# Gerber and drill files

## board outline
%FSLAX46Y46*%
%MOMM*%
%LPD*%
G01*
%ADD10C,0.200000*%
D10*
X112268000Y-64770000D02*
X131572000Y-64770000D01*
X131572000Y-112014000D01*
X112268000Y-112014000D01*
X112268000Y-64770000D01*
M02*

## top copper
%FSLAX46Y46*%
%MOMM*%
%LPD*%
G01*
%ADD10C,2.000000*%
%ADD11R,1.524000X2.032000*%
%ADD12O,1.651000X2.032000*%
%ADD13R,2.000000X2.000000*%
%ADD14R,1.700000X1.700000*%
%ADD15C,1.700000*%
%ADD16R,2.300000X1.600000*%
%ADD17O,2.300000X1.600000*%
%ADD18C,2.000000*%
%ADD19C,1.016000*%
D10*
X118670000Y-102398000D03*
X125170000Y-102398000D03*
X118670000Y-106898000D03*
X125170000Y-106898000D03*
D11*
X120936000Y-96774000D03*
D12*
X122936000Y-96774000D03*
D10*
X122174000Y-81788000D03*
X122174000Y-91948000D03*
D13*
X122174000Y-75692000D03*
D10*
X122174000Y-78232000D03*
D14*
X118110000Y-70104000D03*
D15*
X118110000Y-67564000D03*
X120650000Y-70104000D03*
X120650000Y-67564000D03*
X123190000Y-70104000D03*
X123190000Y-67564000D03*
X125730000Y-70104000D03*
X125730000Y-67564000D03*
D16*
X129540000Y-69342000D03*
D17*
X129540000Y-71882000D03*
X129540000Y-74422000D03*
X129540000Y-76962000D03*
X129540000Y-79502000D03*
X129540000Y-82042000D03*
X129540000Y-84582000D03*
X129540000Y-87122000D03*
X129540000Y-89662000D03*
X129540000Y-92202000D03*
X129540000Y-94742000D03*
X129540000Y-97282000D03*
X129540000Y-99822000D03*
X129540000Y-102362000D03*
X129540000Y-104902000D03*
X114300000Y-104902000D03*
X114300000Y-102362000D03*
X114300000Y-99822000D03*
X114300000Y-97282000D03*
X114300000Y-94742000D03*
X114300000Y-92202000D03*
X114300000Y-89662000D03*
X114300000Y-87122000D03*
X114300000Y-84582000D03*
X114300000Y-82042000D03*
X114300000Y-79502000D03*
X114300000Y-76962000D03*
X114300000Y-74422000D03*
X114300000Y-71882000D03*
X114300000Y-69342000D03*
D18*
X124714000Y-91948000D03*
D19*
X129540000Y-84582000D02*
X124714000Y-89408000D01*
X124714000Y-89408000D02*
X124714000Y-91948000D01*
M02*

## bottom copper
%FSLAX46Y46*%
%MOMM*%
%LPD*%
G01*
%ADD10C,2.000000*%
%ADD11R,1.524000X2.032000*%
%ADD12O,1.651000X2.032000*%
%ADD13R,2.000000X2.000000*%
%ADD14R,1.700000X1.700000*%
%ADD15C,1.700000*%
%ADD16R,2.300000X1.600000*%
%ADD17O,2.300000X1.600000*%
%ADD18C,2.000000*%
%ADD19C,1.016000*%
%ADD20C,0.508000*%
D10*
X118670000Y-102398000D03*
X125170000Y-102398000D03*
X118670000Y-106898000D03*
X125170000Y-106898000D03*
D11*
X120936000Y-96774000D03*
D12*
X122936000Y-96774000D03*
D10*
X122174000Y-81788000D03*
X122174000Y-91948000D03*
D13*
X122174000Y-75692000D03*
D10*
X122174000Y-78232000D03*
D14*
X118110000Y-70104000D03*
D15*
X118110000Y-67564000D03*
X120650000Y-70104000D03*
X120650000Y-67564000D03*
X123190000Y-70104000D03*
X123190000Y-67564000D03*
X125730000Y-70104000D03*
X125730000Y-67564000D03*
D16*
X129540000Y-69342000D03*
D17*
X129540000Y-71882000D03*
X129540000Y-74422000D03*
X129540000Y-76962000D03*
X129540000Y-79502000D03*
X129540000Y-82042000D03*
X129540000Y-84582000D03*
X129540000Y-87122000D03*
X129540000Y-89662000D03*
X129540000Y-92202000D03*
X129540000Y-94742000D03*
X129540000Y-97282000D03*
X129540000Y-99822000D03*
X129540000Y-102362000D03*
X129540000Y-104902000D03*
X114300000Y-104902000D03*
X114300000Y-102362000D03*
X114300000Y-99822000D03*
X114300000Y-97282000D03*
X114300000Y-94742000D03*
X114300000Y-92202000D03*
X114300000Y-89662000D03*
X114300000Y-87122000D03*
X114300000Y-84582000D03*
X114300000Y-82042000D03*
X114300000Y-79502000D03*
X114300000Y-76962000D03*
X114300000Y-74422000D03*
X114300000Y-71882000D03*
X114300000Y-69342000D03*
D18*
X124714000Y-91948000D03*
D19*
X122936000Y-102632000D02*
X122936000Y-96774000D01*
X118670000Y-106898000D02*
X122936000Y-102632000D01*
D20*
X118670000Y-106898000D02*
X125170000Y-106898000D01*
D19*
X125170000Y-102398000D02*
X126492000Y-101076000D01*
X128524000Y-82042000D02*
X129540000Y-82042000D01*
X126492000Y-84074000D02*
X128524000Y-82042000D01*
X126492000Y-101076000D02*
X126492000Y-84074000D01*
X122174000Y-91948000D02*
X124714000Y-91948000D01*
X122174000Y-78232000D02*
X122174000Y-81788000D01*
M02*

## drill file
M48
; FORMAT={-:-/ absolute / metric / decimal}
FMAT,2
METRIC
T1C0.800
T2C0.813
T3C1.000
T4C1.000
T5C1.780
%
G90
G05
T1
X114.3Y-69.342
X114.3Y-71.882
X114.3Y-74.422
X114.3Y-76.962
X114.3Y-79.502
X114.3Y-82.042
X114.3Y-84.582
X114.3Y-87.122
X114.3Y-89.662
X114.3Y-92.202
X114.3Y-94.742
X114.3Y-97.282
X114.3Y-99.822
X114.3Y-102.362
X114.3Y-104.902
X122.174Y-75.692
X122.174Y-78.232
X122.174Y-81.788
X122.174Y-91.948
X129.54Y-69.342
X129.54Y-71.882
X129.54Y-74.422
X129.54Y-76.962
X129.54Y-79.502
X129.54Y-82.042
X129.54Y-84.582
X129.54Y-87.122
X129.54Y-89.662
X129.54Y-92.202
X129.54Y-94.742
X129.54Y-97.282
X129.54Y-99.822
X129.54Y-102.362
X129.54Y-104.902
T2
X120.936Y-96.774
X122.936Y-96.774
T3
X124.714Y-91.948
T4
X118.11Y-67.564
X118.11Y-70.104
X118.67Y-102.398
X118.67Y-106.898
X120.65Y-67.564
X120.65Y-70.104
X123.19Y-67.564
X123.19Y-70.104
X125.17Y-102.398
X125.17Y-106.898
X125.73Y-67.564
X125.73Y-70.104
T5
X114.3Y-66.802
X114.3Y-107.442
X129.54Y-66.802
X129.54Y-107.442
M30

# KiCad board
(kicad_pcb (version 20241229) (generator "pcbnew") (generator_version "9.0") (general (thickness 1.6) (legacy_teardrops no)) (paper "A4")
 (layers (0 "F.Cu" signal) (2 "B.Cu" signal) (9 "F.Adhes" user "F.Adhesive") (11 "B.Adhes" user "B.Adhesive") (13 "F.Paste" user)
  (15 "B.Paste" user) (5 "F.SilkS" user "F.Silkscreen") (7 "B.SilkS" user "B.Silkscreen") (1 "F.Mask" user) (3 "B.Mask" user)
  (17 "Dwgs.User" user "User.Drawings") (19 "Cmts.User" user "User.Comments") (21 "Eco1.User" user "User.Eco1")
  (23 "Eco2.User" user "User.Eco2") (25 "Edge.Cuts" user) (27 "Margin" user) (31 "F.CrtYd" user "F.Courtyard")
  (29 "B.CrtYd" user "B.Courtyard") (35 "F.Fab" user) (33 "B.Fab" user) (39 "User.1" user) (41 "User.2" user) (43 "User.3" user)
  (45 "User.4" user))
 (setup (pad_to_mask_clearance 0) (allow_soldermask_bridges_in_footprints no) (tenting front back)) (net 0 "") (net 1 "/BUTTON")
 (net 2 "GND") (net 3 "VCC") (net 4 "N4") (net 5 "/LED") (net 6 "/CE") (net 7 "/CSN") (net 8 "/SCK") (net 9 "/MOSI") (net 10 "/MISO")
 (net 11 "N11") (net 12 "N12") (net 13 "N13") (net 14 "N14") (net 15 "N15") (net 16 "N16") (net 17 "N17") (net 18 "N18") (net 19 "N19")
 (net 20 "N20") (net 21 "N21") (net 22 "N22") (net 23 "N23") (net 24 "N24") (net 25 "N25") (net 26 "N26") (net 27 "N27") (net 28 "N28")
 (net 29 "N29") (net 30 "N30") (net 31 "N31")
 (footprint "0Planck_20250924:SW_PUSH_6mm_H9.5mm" (layer "F.Cu") (at 118.67 102.398)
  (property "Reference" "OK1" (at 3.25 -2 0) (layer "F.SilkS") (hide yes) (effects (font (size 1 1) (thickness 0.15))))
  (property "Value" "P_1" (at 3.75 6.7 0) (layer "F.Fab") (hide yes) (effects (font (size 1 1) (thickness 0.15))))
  (pad "1" thru_hole circle (at 0 0) (size 2 2) (drill 1) (layers "*.Cu" "*.Mask") (remove_unused_layers no) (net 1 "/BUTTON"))
  (pad "1" thru_hole circle (at 6.5 0) (size 2 2) (drill 1) (layers "*.Cu" "*.Mask") (remove_unused_layers no) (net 1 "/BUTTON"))
  (pad "2" thru_hole circle (at 0 4.5) (size 2 2) (drill 1) (layers "*.Cu" "*.Mask") (remove_unused_layers no) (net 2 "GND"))
  (pad "2" thru_hole circle (at 6.5 4.5) (size 2 2) (drill 1) (layers "*.Cu" "*.Mask") (remove_unused_layers no) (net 2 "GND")))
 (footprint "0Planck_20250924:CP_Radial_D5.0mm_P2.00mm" (layer "F.Cu") (at 120.936 96.774)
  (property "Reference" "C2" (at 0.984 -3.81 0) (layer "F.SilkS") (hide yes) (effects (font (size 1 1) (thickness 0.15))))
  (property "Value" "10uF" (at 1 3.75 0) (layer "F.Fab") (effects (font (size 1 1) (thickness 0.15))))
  (pad "1" thru_hole rect (at 0 0) (size 1.524 2.032) (drill 0.8128) (layers "*.Cu" "*.Mask") (remove_unused_layers no) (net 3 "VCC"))
  (pad "2" thru_hole oval (at 2 0) (size 1.651 2.032) (drill 0.8128) (layers "*.Cu" "*.Mask") (remove_unused_layers no) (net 2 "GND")))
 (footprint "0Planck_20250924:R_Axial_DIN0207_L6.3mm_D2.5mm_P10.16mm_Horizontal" (layer "F.Cu") (at 122.174 81.788 -90)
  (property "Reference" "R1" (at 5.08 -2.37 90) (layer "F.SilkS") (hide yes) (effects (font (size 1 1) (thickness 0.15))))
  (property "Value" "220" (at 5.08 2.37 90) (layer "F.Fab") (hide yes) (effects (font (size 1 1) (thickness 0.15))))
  (pad "1" thru_hole circle (at 0 0 270) (size 2 2) (drill 0.8) (layers "*.Cu" "*.Mask") (remove_unused_layers no) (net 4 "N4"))
  (pad "2" thru_hole circle (at 10.16 0 270) (size 2 2) (drill 0.8) (layers "*.Cu" "*.Mask") (remove_unused_layers no) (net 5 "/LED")))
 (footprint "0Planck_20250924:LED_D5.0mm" (layer "F.Cu") (at 122.174 75.692 -90)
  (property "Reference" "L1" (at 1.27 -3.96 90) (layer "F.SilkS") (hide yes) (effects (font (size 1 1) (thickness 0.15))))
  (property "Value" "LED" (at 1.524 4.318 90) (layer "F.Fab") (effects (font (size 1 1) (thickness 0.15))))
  (pad "1" thru_hole rect (at 0 0 270) (size 2 2) (drill 0.8) (layers "*.Cu" "*.Mask") (remove_unused_layers no) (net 2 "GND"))
  (pad "2" thru_hole circle (at 2.54 0 270) (size 2 2) (drill 0.8) (layers "*.Cu" "*.Mask") (remove_unused_layers no) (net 4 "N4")))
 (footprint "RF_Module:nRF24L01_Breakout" (layer "F.Cu") (at 118.11 70.104 90)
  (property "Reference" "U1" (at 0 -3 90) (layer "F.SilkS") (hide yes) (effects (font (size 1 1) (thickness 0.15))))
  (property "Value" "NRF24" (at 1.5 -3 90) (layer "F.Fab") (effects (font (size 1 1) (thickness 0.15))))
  (pad "1" thru_hole rect (at 0 0 90) (size 1.7 1.7) (drill 1) (layers "*.Cu" "*.Mask") (remove_unused_layers no) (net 2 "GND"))
  (pad "2" thru_hole circle (at 2.54 0 90) (size 1.7 1.7) (drill 1) (layers "*.Cu" "*.Mask") (remove_unused_layers no) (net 3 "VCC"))
  (pad "3" thru_hole circle (at 0 2.54 90) (size 1.7 1.7) (drill 1) (layers "*.Cu" "*.Mask") (remove_unused_layers no) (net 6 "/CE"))
  (pad "4" thru_hole circle (at 2.54 2.54 90) (size 1.7 1.7) (drill 1) (layers "*.Cu" "*.Mask") (remove_unused_layers no) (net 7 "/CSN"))
  (pad "5" thru_hole circle (at 0 5.08 90) (size 1.7 1.7) (drill 1) (layers "*.Cu" "*.Mask") (remove_unused_layers no) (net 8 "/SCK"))
  (pad "6" thru_hole circle (at 2.54 5.08 90) (size 1.7 1.7) (drill 1) (layers "*.Cu" "*.Mask") (remove_unused_layers no) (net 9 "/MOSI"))
  (pad "7" thru_hole circle (at 0 7.62 90) (size 1.7 1.7) (drill 1) (layers "*.Cu" "*.Mask") (remove_unused_layers no) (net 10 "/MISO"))
  (pad "8" thru_hole circle (at 2.54 7.62 90) (size 1.7 1.7) (drill 1) (layers "*.Cu" "*.Mask") (remove_unused_layers no) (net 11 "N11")))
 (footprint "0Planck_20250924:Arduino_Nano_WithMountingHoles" (layer "B.Cu") (at 129.54 69.342 180)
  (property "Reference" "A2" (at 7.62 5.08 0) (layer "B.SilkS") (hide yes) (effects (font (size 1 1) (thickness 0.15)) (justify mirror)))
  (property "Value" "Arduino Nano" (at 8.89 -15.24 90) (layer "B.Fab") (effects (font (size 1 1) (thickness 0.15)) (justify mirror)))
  (pad "" np_thru_hole circle (at 0 -38.1 180) (size 1.78 1.78) (drill 1.78) (layers "*.Cu" "*.Mask"))
  (pad "" np_thru_hole circle (at 0 2.54 180) (size 1.78 1.78) (drill 1.78) (layers "*.Cu" "*.Mask"))
  (pad "" np_thru_hole circle (at 15.24 -38.1 180) (size 1.78 1.78) (drill 1.78) (layers "*.Cu" "*.Mask"))
  (pad "" np_thru_hole circle (at 15.24 2.54 180) (size 1.78 1.78) (drill 1.78) (layers "*.Cu" "*.Mask"))
  (pad "1" thru_hole rect (at 0 0 180) (size 2.3 1.6) (drill 0.8) (layers "*.Cu" "*.Mask") (remove_unused_layers no) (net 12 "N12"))
  (pad "2" thru_hole oval (at 0 -2.54 180) (size 2.3 1.6) (drill 0.8) (layers "*.Cu" "*.Mask") (remove_unused_layers no) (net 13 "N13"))
  (pad "3" thru_hole oval (at 0 -5.08 180) (size 2.3 1.6) (drill 0.8) (layers "*.Cu" "*.Mask") (remove_unused_layers no) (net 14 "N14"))
  (pad "4" thru_hole oval (at 0 -7.62 180) (size 2.3 1.6) (drill 0.8) (layers "*.Cu" "*.Mask") (remove_unused_layers no) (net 2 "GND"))
  (pad "5" thru_hole oval (at 0 -10.16 180) (size 2.3 1.6) (drill 0.8) (layers "*.Cu" "*.Mask") (remove_unused_layers no) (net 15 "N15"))
  (pad "6" thru_hole oval (at 0 -12.7 180) (size 2.3 1.6) (drill 0.8) (layers "*.Cu" "*.Mask") (remove_unused_layers no) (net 1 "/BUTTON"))
  (pad "7" thru_hole oval (at 0 -15.24 180) (size 2.3 1.6) (drill 0.8) (layers "*.Cu" "*.Mask") (remove_unused_layers no) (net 5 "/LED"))
  (pad "8" thru_hole oval (at 0 -17.78 180) (size 2.3 1.6) (drill 0.8) (layers "*.Cu" "*.Mask") (remove_unused_layers no) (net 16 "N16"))
  (pad "9" thru_hole oval (at 0 -20.32 180) (size 2.3 1.6) (drill 0.8) (layers "*.Cu" "*.Mask") (remove_unused_layers no) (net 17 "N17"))
  (pad "10" thru_hole oval (at 0 -22.86 180) (size 2.3 1.6) (drill 0.8) (layers "*.Cu" "*.Mask") (remove_unused_layers no) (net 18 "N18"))
  (pad "11" thru_hole oval (at 0 -25.4 180) (size 2.3 1.6) (drill 0.8) (layers "*.Cu" "*.Mask") (remove_unused_layers no) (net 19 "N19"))
  (pad "12" thru_hole oval (at 0 -27.94 180) (size 2.3 1.6) (drill 0.8) (layers "*.Cu" "*.Mask") (remove_unused_layers no) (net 6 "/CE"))
  (pad "13" thru_hole oval (at 0 -30.48 180) (size 2.3 1.6) (drill 0.8) (layers "*.Cu" "*.Mask") (remove_unused_layers no) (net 7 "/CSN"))
  (pad "14" thru_hole oval (at 0 -33.02 180) (size 2.3 1.6) (drill 0.8) (layers "*.Cu" "*.Mask") (remove_unused_layers no) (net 9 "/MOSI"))
  (pad "15" thru_hole oval (at 0 -35.56 180) (size 2.3 1.6) (drill 0.8) (layers "*.Cu" "*.Mask") (remove_unused_layers no) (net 10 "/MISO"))
  (pad "16" thru_hole oval (at 15.24 -35.56 180) (size 2.3 1.6) (drill 0.8) (layers "*.Cu" "*.Mask") (remove_unused_layers no)
   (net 8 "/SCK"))
  (pad "17" thru_hole oval (at 15.24 -33.02 180) (size 2.3 1.6) (drill 0.8) (layers "*.Cu" "*.Mask") (remove_unused_layers no) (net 3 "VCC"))
  (pad "18" thru_hole oval (at 15.24 -30.48 180) (size 2.3 1.6) (drill 0.8) (layers "*.Cu" "*.Mask") (remove_unused_layers no)
   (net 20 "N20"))
  (pad "19" thru_hole oval (at 15.24 -27.94 180) (size 2.3 1.6) (drill 0.8) (layers "*.Cu" "*.Mask") (remove_unused_layers no)
   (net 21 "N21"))
  (pad "20" thru_hole oval (at 15.24 -25.4 180) (size 2.3 1.6) (drill 0.8) (layers "*.Cu" "*.Mask") (remove_unused_layers no) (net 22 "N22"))
  (pad "21" thru_hole oval (at 15.24 -22.86 180) (size 2.3 1.6) (drill 0.8) (layers "*.Cu" "*.Mask") (remove_unused_layers no)
   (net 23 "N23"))
  (pad "22" thru_hole oval (at 15.24 -20.32 180) (size 2.3 1.6) (drill 0.8) (layers "*.Cu" "*.Mask") (remove_unused_layers no)
   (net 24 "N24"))
  (pad "23" thru_hole oval (at 15.24 -17.78 180) (size 2.3 1.6) (drill 0.8) (layers "*.Cu" "*.Mask") (remove_unused_layers no)
   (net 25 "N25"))
  (pad "24" thru_hole oval (at 15.24 -15.24 180) (size 2.3 1.6) (drill 0.8) (layers "*.Cu" "*.Mask") (remove_unused_layers no)
   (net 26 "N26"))
  (pad "25" thru_hole oval (at 15.24 -12.7 180) (size 2.3 1.6) (drill 0.8) (layers "*.Cu" "*.Mask") (remove_unused_layers no) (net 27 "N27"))
  (pad "26" thru_hole oval (at 15.24 -10.16 180) (size 2.3 1.6) (drill 0.8) (layers "*.Cu" "*.Mask") (remove_unused_layers no)
   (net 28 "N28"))
  (pad "27" thru_hole oval (at 15.24 -7.62 180) (size 2.3 1.6) (drill 0.8) (layers "*.Cu" "*.Mask") (remove_unused_layers no) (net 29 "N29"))
  (pad "28" thru_hole oval (at 15.24 -5.08 180) (size 2.3 1.6) (drill 0.8) (layers "*.Cu" "*.Mask") (remove_unused_layers no) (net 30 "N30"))
  (pad "29" thru_hole oval (at 15.24 -2.54 180) (size 2.3 1.6) (drill 0.8) (layers "*.Cu" "*.Mask") (remove_unused_layers no) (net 2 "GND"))
  (pad "30" thru_hole oval (at 15.24 0 180) (size 2.3 1.6) (drill 0.8) (layers "*.Cu" "*.Mask") (remove_unused_layers no) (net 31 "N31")))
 (gr_rect (start 112.268 64.77) (end 131.572 112.014) (stroke (width 0.2) (type solid)) (fill no) (layer "Edge.Cuts"))
 (segment (start 122.936 102.632) (end 122.936 96.774) (width 1.016) (layer "B.Cu") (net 2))
 (segment (start 118.67 106.898) (end 122.936 102.632) (width 1.016) (layer "B.Cu") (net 2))
 (segment (start 118.67 106.898) (end 125.17 106.898) (width 0.508) (layer "B.Cu") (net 2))
 (segment (start 125.17 102.398) (end 126.492 101.076) (width 1.016) (layer "B.Cu") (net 1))
 (segment (start 128.524 82.042) (end 129.54 82.042) (width 1.016) (layer "B.Cu") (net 1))
 (segment (start 126.492 84.074) (end 128.524 82.042) (width 1.016) (layer "B.Cu") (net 1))
 (segment (start 126.492 101.076) (end 126.492 84.074) (width 1.016) (layer "B.Cu") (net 1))
 (segment (start 129.54 84.582) (end 124.714 89.408) (width 1.016) (layer "F.Cu") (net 5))
 (segment (start 124.714 89.408) (end 124.714 91.948) (width 1.016) (layer "F.Cu") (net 5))
 (via (at 124.714 91.948) (size 2) (drill 1) (layers "F.Cu" "B.Cu") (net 5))
 (segment (start 122.174 91.948) (end 124.714 91.948) (width 1.016) (layer "B.Cu") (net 5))
 (segment (start 122.174 78.232) (end 122.174 81.788) (width 1.016) (layer "B.Cu") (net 4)))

